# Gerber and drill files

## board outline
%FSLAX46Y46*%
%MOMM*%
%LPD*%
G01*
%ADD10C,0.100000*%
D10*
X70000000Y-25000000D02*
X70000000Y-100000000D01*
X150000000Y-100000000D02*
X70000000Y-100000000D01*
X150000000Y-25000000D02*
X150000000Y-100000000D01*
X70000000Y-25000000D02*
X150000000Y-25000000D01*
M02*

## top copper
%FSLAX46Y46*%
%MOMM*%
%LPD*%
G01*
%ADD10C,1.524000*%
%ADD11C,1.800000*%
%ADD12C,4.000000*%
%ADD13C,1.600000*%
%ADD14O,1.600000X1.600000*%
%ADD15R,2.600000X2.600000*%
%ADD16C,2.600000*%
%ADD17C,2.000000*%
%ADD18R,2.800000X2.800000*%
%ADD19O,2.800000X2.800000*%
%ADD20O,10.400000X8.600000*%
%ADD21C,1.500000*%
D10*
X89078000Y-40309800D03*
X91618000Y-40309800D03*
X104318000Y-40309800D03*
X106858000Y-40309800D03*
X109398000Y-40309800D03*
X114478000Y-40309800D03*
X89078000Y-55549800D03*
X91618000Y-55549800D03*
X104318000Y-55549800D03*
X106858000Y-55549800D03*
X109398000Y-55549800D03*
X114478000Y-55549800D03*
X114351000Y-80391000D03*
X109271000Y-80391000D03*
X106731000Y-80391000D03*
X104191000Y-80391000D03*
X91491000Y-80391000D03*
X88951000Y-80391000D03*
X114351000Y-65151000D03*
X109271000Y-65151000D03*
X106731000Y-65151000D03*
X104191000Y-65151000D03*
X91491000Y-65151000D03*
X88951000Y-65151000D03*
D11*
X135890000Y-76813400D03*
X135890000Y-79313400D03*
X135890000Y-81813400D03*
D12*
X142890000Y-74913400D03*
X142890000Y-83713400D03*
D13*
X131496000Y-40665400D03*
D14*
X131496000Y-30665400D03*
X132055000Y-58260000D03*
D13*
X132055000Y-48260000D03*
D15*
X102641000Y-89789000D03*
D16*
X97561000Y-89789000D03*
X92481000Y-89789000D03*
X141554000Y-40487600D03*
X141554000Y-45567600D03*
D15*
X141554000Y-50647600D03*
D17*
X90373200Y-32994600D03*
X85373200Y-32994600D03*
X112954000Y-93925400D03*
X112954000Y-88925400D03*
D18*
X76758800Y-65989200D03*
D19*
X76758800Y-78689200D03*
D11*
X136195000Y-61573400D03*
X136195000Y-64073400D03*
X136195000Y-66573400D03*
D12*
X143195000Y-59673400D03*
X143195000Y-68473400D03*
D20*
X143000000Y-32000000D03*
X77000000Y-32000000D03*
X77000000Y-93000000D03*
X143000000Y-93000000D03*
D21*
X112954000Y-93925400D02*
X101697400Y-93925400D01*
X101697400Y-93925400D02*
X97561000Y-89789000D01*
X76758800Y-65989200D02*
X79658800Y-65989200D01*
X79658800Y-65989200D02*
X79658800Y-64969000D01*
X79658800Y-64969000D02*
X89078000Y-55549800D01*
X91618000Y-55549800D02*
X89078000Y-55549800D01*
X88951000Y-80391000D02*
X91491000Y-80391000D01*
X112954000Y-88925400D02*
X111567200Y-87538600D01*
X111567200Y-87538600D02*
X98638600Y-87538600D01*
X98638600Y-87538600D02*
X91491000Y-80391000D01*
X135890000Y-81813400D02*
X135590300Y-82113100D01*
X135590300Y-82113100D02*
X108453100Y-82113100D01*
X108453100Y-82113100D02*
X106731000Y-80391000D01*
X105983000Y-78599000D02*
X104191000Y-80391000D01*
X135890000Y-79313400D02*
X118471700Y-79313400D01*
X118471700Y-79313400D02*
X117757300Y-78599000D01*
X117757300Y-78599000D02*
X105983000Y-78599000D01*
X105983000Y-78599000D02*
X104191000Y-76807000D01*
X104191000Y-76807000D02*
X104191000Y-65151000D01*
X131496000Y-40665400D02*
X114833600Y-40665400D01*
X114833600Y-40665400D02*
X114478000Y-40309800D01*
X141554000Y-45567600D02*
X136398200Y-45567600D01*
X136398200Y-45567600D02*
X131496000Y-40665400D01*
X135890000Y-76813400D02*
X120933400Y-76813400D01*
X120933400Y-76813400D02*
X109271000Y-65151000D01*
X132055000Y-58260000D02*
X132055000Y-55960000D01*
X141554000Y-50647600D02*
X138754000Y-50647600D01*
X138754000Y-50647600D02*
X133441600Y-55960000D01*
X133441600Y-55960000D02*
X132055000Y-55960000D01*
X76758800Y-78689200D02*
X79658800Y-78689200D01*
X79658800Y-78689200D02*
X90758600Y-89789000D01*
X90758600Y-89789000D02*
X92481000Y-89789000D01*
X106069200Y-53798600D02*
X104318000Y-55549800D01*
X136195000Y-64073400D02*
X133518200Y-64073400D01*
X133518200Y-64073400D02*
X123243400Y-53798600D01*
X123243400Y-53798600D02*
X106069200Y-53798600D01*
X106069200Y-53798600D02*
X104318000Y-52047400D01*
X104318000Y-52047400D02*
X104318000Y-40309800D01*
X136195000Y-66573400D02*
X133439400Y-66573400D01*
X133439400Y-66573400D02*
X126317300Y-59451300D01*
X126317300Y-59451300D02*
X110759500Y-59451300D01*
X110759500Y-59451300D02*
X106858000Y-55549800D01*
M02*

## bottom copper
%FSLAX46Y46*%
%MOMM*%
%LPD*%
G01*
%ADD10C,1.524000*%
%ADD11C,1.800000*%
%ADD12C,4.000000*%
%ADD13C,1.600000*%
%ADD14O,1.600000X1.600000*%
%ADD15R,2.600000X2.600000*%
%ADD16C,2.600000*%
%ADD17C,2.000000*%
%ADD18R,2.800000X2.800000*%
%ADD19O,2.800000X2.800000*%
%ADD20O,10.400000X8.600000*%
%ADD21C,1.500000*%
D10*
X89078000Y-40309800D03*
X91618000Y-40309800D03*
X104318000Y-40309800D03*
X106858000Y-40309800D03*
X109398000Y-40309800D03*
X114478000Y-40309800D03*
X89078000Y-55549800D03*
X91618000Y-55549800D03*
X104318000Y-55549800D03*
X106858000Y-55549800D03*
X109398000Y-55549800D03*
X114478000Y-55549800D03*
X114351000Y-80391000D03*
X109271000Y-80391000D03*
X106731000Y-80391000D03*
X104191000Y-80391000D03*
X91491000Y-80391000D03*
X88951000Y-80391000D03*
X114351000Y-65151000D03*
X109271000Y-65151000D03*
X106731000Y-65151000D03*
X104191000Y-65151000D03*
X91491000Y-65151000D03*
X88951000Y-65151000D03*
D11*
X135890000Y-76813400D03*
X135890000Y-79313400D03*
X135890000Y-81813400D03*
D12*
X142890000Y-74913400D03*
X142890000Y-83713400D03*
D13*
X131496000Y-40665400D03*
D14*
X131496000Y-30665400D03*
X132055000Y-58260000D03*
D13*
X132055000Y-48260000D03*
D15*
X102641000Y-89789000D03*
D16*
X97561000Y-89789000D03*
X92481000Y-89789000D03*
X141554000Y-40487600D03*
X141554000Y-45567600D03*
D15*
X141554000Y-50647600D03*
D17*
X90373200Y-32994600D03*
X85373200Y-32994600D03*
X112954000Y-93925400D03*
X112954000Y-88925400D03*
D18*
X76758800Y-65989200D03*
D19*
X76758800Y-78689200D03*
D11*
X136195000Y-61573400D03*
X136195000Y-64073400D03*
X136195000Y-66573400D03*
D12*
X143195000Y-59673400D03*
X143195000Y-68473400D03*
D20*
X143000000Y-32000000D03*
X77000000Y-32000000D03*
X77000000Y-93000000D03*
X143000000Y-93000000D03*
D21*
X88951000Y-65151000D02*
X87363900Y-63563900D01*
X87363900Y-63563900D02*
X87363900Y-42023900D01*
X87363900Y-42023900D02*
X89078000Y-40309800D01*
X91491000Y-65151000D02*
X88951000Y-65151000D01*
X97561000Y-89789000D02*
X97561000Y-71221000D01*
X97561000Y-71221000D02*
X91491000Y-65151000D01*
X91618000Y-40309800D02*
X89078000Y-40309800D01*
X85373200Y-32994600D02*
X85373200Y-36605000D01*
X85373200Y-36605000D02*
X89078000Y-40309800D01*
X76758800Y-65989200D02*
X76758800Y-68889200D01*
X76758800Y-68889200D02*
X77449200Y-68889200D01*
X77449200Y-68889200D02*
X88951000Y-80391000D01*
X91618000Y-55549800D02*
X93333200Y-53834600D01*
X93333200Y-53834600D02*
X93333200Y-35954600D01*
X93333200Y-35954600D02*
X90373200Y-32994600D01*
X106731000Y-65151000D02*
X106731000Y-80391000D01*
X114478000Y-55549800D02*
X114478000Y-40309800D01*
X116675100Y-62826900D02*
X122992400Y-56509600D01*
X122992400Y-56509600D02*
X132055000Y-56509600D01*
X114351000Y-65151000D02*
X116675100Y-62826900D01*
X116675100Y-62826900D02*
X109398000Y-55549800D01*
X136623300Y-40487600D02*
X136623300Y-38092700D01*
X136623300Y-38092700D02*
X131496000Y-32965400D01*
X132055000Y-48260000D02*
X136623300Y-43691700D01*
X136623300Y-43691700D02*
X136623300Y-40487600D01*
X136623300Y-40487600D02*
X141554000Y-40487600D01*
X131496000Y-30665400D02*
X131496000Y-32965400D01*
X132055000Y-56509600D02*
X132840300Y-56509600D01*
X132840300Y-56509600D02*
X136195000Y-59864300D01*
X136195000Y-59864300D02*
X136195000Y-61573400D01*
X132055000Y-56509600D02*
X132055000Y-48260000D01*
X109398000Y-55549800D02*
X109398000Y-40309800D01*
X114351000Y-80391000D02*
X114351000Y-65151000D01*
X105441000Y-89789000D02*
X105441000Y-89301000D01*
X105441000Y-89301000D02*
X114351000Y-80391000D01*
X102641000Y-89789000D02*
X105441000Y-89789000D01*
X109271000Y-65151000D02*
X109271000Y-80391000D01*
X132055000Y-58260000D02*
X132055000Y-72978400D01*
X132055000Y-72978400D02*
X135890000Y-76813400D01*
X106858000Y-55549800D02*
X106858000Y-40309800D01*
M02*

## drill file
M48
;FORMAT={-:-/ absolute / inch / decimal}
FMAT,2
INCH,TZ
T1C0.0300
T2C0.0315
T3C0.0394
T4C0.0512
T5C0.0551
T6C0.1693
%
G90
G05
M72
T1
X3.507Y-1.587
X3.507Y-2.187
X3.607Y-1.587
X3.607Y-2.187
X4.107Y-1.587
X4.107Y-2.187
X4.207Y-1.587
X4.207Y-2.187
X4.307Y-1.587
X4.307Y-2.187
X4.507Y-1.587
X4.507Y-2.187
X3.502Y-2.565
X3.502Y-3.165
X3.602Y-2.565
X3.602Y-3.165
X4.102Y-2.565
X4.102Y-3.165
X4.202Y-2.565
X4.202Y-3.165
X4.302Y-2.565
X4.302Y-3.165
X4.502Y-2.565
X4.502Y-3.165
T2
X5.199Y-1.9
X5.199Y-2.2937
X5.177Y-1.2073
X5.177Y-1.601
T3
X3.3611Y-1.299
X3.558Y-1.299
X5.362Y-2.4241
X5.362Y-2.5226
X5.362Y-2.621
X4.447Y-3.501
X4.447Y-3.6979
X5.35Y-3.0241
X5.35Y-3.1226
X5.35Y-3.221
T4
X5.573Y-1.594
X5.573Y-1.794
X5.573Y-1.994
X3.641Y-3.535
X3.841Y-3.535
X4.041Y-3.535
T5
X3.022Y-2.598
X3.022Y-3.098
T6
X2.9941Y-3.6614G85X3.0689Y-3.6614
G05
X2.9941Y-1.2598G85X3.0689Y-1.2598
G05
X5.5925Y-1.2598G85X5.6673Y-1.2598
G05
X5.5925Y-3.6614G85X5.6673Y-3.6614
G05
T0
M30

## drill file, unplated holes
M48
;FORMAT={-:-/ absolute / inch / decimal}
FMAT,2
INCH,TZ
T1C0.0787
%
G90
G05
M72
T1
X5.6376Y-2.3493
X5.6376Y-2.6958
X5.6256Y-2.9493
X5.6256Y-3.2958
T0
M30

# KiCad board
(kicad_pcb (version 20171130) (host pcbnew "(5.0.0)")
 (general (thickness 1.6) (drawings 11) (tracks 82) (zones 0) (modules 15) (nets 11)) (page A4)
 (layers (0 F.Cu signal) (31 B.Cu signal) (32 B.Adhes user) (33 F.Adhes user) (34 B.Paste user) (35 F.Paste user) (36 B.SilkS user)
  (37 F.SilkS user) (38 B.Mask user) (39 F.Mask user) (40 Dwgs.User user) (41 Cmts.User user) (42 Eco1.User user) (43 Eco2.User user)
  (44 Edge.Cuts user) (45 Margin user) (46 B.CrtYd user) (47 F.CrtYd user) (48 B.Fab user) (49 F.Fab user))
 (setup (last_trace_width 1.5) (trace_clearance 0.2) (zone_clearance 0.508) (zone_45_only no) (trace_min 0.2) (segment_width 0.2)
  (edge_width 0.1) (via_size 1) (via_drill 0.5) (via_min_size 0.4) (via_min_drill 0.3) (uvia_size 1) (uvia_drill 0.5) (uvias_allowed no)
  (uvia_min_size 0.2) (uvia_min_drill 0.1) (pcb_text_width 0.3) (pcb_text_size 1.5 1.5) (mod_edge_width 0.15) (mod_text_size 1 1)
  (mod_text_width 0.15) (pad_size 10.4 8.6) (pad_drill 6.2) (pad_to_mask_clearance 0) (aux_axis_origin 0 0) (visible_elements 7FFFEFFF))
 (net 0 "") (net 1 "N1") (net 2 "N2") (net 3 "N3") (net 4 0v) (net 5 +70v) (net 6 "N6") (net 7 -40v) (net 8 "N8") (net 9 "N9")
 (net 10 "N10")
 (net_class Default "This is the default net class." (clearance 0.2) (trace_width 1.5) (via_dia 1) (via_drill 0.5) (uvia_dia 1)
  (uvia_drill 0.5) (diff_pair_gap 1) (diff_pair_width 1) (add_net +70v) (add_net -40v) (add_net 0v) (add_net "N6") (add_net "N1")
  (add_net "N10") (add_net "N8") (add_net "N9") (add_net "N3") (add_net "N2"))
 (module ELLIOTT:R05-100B (layer F.Cu) (at 101.778 47.9298)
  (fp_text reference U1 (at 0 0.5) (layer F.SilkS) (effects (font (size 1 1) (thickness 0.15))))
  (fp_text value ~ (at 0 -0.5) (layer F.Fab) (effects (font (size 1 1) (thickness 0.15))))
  (pad 2 thru_hole circle (at -12.7 -7.62) (size 1.524 1.524) (drill 0.762) (layers *.Cu *.Mask) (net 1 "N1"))
  (pad 3 thru_hole circle (at -10.16 -7.62) (size 1.524 1.524) (drill 0.762) (layers *.Cu *.Mask) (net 1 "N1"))
  (pad 8 thru_hole circle (at 2.54 -7.62) (size 1.524 1.524) (drill 0.762) (layers *.Cu *.Mask) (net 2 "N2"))
  (pad 9 thru_hole circle (at 5.08 -7.62) (size 1.524 1.524) (drill 0.762) (layers *.Cu *.Mask) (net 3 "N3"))
  (pad 10 thru_hole circle (at 7.62 -7.62) (size 1.524 1.524) (drill 0.762) (layers *.Cu *.Mask) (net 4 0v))
  (pad 12 thru_hole circle (at 12.7 -7.62) (size 1.524 1.524) (drill 0.762) (layers *.Cu *.Mask) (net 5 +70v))
  (pad 22 thru_hole circle (at -12.7 7.62) (size 1.524 1.524) (drill 0.762) (layers *.Cu *.Mask) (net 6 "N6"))
  (pad 23 thru_hole circle (at -10.16 7.62) (size 1.524 1.524) (drill 0.762) (layers *.Cu *.Mask) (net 6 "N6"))
  (pad 17 thru_hole circle (at 2.54 7.62) (size 1.524 1.524) (drill 0.762) (layers *.Cu *.Mask) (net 2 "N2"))
  (pad 16 thru_hole circle (at 5.08 7.62) (size 1.524 1.524) (drill 0.762) (layers *.Cu *.Mask) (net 3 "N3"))
  (pad 15 thru_hole circle (at 7.62 7.62) (size 1.524 1.524) (drill 0.762) (layers *.Cu *.Mask) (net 4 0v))
  (pad 13 thru_hole circle (at 12.7 7.62) (size 1.524 1.524) (drill 0.762) (layers *.Cu *.Mask) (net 5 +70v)))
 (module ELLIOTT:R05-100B (layer F.Cu) (at 101.651 72.771)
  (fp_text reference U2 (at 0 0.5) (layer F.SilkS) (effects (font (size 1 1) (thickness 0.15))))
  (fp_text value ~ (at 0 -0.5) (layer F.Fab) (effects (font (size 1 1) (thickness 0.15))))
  (pad 13 thru_hole circle (at 12.7 7.62) (size 1.524 1.524) (drill 0.762) (layers *.Cu *.Mask) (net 4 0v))
  (pad 15 thru_hole circle (at 7.62 7.62) (size 1.524 1.524) (drill 0.762) (layers *.Cu *.Mask) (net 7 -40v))
  (pad 16 thru_hole circle (at 5.08 7.62) (size 1.524 1.524) (drill 0.762) (layers *.Cu *.Mask) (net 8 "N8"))
  (pad 17 thru_hole circle (at 2.54 7.62) (size 1.524 1.524) (drill 0.762) (layers *.Cu *.Mask) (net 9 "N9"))
  (pad 23 thru_hole circle (at -10.16 7.62) (size 1.524 1.524) (drill 0.762) (layers *.Cu *.Mask) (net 6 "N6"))
  (pad 22 thru_hole circle (at -12.7 7.62) (size 1.524 1.524) (drill 0.762) (layers *.Cu *.Mask) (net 6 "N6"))
  (pad 12 thru_hole circle (at 12.7 -7.62) (size 1.524 1.524) (drill 0.762) (layers *.Cu *.Mask) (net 4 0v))
  (pad 10 thru_hole circle (at 7.62 -7.62) (size 1.524 1.524) (drill 0.762) (layers *.Cu *.Mask) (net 7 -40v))
  (pad 9 thru_hole circle (at 5.08 -7.62) (size 1.524 1.524) (drill 0.762) (layers *.Cu *.Mask) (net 8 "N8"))
  (pad 8 thru_hole circle (at 2.54 -7.62) (size 1.524 1.524) (drill 0.762) (layers *.Cu *.Mask) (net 9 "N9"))
  (pad 3 thru_hole circle (at -10.16 -7.62) (size 1.524 1.524) (drill 0.762) (layers *.Cu *.Mask) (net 1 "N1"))
  (pad 2 thru_hole circle (at -12.7 -7.62) (size 1.524 1.524) (drill 0.762) (layers *.Cu *.Mask) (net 1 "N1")))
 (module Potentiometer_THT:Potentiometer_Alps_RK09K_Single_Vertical (layer F.Cu) (at 135.89 81.8134)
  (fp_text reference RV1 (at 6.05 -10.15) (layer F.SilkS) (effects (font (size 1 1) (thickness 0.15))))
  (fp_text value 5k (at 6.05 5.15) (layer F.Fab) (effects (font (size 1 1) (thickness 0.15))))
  (pad 3 thru_hole circle (at 0 -5) (size 1.8 1.8) (drill 1) (layers *.Cu *.Mask) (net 7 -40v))
  (pad 2 thru_hole circle (at 0 -2.5) (size 1.8 1.8) (drill 1) (layers *.Cu *.Mask) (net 9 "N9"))
  (pad 1 thru_hole circle (at 0 0) (size 1.8 1.8) (drill 1) (layers *.Cu *.Mask) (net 8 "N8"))
  (pad "" np_thru_hole circle (at 7 -6.9) (size 4 4) (drill 2) (layers *.Cu *.Mask))
  (pad "" np_thru_hole circle (at 7 1.9) (size 4 4) (drill 2) (layers *.Cu *.Mask)))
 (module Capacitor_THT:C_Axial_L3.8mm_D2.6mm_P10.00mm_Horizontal (layer F.Cu) (at 131.496 40.6654 90)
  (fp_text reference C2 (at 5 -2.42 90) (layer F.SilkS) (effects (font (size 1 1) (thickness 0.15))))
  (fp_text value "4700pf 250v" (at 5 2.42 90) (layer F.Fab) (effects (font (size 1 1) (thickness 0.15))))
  (pad 1 thru_hole circle (at 0 0 90) (size 1.6 1.6) (drill 0.8) (layers *.Cu *.Mask) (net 5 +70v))
  (pad 2 thru_hole oval (at 10 0 90) (size 1.6 1.6) (drill 0.8) (layers *.Cu *.Mask) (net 4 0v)))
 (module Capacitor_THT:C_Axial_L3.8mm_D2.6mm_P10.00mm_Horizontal (layer F.Cu) (at 132.055 48.26 270)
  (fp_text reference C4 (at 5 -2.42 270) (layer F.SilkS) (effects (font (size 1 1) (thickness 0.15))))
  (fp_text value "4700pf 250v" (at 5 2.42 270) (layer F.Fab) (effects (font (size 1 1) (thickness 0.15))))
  (pad 2 thru_hole oval (at 10 0 270) (size 1.6 1.6) (drill 0.8) (layers *.Cu *.Mask) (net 7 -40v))
  (pad 1 thru_hole circle (at 0 0 270) (size 1.6 1.6) (drill 0.8) (layers *.Cu *.Mask) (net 4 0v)))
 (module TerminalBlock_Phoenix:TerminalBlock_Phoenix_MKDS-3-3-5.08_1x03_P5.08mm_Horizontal (layer F.Cu) (at 102.641 89.789 180)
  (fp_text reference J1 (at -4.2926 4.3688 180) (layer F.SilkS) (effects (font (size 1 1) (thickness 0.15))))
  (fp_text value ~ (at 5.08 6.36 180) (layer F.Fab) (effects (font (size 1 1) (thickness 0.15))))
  (pad 1 thru_hole rect (at 0 0 180) (size 2.6 2.6) (drill 1.3) (layers *.Cu *.Mask) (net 4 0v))
  (pad 2 thru_hole circle (at 5.08 0 180) (size 2.6 2.6) (drill 1.3) (layers *.Cu *.Mask) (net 1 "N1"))
  (pad 3 thru_hole circle (at 10.16 0 180) (size 2.6 2.6) (drill 1.3) (layers *.Cu *.Mask) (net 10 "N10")))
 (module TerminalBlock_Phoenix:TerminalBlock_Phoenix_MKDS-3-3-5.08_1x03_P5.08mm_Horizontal (layer F.Cu) (at 141.554 50.6476 90)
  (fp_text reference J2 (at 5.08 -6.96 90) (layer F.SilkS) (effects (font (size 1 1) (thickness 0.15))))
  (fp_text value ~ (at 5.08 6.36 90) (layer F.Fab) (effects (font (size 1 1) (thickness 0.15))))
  (pad 3 thru_hole circle (at 10.16 0 90) (size 2.6 2.6) (drill 1.3) (layers *.Cu *.Mask) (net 4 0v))
  (pad 2 thru_hole circle (at 5.08 0 90) (size 2.6 2.6) (drill 1.3) (layers *.Cu *.Mask) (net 5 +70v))
  (pad 1 thru_hole rect (at 0 0 90) (size 2.6 2.6) (drill 1.3) (layers *.Cu *.Mask) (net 7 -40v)))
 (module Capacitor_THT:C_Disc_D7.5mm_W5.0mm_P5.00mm (layer F.Cu) (at 90.3732 32.9946 180)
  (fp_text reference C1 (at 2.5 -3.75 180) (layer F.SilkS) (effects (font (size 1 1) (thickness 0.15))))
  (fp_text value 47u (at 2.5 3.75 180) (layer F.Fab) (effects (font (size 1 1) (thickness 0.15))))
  (pad 1 thru_hole circle (at 0 0 180) (size 2 2) (drill 1) (layers *.Cu *.Mask) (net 6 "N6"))
  (pad 2 thru_hole circle (at 5 0 180) (size 2 2) (drill 1) (layers *.Cu *.Mask) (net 1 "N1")))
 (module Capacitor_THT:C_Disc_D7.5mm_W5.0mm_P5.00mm (layer F.Cu) (at 112.954 88.9254 270)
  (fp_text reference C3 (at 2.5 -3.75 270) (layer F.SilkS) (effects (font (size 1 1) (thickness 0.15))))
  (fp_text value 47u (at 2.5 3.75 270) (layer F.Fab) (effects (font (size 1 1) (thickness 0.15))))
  (pad 2 thru_hole circle (at 5 0 270) (size 2 2) (drill 1) (layers *.Cu *.Mask) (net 1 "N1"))
  (pad 1 thru_hole circle (at 0 0 270) (size 2 2) (drill 1) (layers *.Cu *.Mask) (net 6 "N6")))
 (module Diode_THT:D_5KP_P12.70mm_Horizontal (layer F.Cu) (at 76.7588 65.9892 270)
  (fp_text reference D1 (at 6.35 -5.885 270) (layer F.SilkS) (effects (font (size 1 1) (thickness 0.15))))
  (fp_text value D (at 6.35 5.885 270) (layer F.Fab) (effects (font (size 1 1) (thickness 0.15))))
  (pad 1 thru_hole rect (at 0 0 270) (size 2.8 2.8) (drill 1.4) (layers *.Cu *.Mask) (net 6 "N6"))
  (pad 2 thru_hole oval (at 12.7 0 270) (size 2.8 2.8) (drill 1.4) (layers *.Cu *.Mask) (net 10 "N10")))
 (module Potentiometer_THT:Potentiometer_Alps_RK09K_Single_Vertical (layer F.Cu) (at 136.195 66.5734)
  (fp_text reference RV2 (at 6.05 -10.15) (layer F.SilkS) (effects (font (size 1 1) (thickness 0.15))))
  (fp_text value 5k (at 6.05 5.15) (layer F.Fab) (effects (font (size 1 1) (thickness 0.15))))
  (pad 3 thru_hole circle (at 0 -5) (size 1.8 1.8) (drill 1) (layers *.Cu *.Mask) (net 4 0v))
  (pad 2 thru_hole circle (at 0 -2.5) (size 1.8 1.8) (drill 1) (layers *.Cu *.Mask) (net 2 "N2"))
  (pad 1 thru_hole circle (at 0 0) (size 1.8 1.8) (drill 1) (layers *.Cu *.Mask) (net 3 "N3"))
  (pad "" np_thru_hole circle (at 7 -6.9) (size 4 4) (drill 2) (layers *.Cu *.Mask))
  (pad "" np_thru_hole circle (at 7 1.9) (size 4 4) (drill 2) (layers *.Cu *.Mask)))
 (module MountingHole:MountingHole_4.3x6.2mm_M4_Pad (layer F.Cu) (at 143 32)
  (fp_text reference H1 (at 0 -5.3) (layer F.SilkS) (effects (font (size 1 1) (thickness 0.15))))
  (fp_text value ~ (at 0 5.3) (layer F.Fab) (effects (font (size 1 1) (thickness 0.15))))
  (pad 1 thru_hole oval (at 0 0) (size 10.4 8.6) (drill oval 6.2 4.3) (layers *.Cu *.Mask)))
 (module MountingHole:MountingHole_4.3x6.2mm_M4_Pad (layer F.Cu) (at 77 32)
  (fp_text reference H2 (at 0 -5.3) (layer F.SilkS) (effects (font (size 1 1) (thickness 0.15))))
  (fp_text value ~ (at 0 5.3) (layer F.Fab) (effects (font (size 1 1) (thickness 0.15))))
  (pad 1 thru_hole oval (at 0 0) (size 10.4 8.6) (drill oval 6.2 4.3) (layers *.Cu *.Mask)))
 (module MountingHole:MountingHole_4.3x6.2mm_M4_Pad (layer F.Cu) (at 77 93)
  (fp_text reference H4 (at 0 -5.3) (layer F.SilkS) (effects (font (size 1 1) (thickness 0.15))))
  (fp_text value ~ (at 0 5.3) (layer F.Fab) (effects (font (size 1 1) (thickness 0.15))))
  (pad 1 thru_hole oval (at 0 0) (size 10.4 8.6) (drill oval 6.2 4.3) (layers *.Cu *.Mask)))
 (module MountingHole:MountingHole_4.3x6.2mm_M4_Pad (layer F.Cu) (at 143 93)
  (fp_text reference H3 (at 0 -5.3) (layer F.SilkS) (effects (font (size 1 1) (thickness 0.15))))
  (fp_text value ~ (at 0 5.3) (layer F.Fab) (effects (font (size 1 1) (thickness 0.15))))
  (pad 1 thru_hole oval (at 0 0) (size 10.4 8.6) (drill oval 6.2 4.3) (layers *.Cu *.Mask)))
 (gr_line (start 70 25) (end 70 100) (layer Edge.Cuts) (width 0.1))
 (gr_line (start 150 100) (end 70 100) (layer Edge.Cuts) (width 0.1))
 (gr_line (start 150 25) (end 150 100) (layer Edge.Cuts) (width 0.1))
 (gr_line (start 70 25) (end 150 25) (layer Edge.Cuts) (width 0.1))
 (segment (start 88.951 65.151) (end 87.3639 63.5639) (width 1.5) (layer B.Cu) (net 1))
 (segment (start 87.3639 63.5639) (end 87.3639 42.0239) (width 1.5) (layer B.Cu) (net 1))
 (segment (start 87.3639 42.0239) (end 89.078 40.3098) (width 1.5) (layer B.Cu) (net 1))
 (segment (start 91.491 65.151) (end 88.951 65.151) (width 1.5) (layer B.Cu) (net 1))
 (segment (start 97.561 89.789) (end 97.561 71.221) (width 1.5) (layer B.Cu) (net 1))
 (segment (start 97.561 71.221) (end 91.491 65.151) (width 1.5) (layer B.Cu) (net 1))
 (segment (start 91.618 40.3098) (end 89.078 40.3098) (width 1.5) (layer B.Cu) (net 1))
 (segment (start 85.3732 32.9946) (end 85.3732 36.605) (width 1.5) (layer B.Cu) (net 1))
 (segment (start 85.3732 36.605) (end 89.078 40.3098) (width 1.5) (layer B.Cu) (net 1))
 (segment (start 112.954 93.9254) (end 101.6974 93.9254) (width 1.5) (layer F.Cu) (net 1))
 (segment (start 101.6974 93.9254) (end 97.561 89.789) (width 1.5) (layer F.Cu) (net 1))
 (segment (start 76.7588 65.9892) (end 76.7588 68.8892) (width 1.5) (layer B.Cu) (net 6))
 (segment (start 76.7588 68.8892) (end 77.4492 68.8892) (width 1.5) (layer B.Cu) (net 6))
 (segment (start 77.4492 68.8892) (end 88.951 80.391) (width 1.5) (layer B.Cu) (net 6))
 (segment (start 91.618 55.5498) (end 93.3332 53.8346) (width 1.5) (layer B.Cu) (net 6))
 (segment (start 93.3332 53.8346) (end 93.3332 35.9546) (width 1.5) (layer B.Cu) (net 6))
 (segment (start 93.3332 35.9546) (end 90.3732 32.9946) (width 1.5) (layer B.Cu) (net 6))
 (segment (start 76.7588 65.9892) (end 79.6588 65.9892) (width 1.5) (layer F.Cu) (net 6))
 (segment (start 79.6588 65.9892) (end 79.6588 64.969) (width 1.5) (layer F.Cu) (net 6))
 (segment (start 79.6588 64.969) (end 89.078 55.5498) (width 1.5) (layer F.Cu) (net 6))
 (segment (start 91.618 55.5498) (end 89.078 55.5498) (width 1.5) (layer F.Cu) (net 6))
 (segment (start 88.951 80.391) (end 91.491 80.391) (width 1.5) (layer F.Cu) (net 6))
 (segment (start 112.954 88.9254) (end 111.5672 87.5386) (width 1.5) (layer F.Cu) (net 6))
 (segment (start 111.5672 87.5386) (end 98.6386 87.5386) (width 1.5) (layer F.Cu) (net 6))
 (segment (start 98.6386 87.5386) (end 91.491 80.391) (width 1.5) (layer F.Cu) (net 6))
 (segment (start 106.731 65.151) (end 106.731 80.391) (width 1.5) (layer B.Cu) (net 8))
 (segment (start 135.89 81.8134) (end 135.5903 82.1131) (width 1.5) (layer F.Cu) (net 8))
 (segment (start 135.5903 82.1131) (end 108.4531 82.1131) (width 1.5) (layer F.Cu) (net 8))
 (segment (start 108.4531 82.1131) (end 106.731 80.391) (width 1.5) (layer F.Cu) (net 8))
 (segment (start 105.983 78.599) (end 104.191 80.391) (width 1.5) (layer F.Cu) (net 9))
 (segment (start 135.89 79.3134) (end 118.4717 79.3134) (width 1.5) (layer F.Cu) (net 9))
 (segment (start 118.4717 79.3134) (end 117.7573 78.599) (width 1.5) (layer F.Cu) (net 9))
 (segment (start 117.7573 78.599) (end 105.983 78.599) (width 1.5) (layer F.Cu) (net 9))
 (segment (start 105.983 78.599) (end 104.191 76.807) (width 1.5) (layer F.Cu) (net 9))
 (segment (start 104.191 76.807) (end 104.191 65.151) (width 1.5) (layer F.Cu) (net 9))
 (segment (start 114.478 55.5498) (end 114.478 40.3098) (width 1.5) (layer B.Cu) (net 5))
 (segment (start 131.496 40.6654) (end 114.8336 40.6654) (width 1.5) (layer F.Cu) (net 5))
 (segment (start 114.8336 40.6654) (end 114.478 40.3098) (width 1.5) (layer F.Cu) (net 5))
 (segment (start 141.554 45.5676) (end 136.3982 45.5676) (width 1.5) (layer F.Cu) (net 5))
 (segment (start 136.3982 45.5676) (end 131.496 40.6654) (width 1.5) (layer F.Cu) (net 5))
 (segment (start 116.6751 62.8269) (end 122.9924 56.5096) (width 1.5) (layer B.Cu) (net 4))
 (segment (start 122.9924 56.5096) (end 132.055 56.5096) (width 1.5) (layer B.Cu) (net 4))
 (segment (start 114.351 65.151) (end 116.6751 62.8269) (width 1.5) (layer B.Cu) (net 4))
 (segment (start 116.6751 62.8269) (end 109.398 55.5498) (width 1.5) (layer B.Cu) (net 4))
 (segment (start 136.6233 40.4876) (end 136.6233 38.0927) (width 1.5) (layer B.Cu) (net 4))
 (segment (start 136.6233 38.0927) (end 131.496 32.9654) (width 1.5) (layer B.Cu) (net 4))
 (segment (start 132.055 48.26) (end 136.6233 43.6917) (width 1.5) (layer B.Cu) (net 4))
 (segment (start 136.6233 43.6917) (end 136.6233 40.4876) (width 1.5) (layer B.Cu) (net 4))
 (segment (start 136.6233 40.4876) (end 141.554 40.4876) (width 1.5) (layer B.Cu) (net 4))
 (segment (start 131.496 30.6654) (end 131.496 32.9654) (width 1.5) (layer B.Cu) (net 4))
 (segment (start 132.055 56.5096) (end 132.8403 56.5096) (width 1.5) (layer B.Cu) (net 4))
 (segment (start 132.8403 56.5096) (end 136.195 59.8643) (width 1.5) (layer B.Cu) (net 4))
 (segment (start 136.195 59.8643) (end 136.195 61.5734) (width 1.5) (layer B.Cu) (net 4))
 (segment (start 132.055 56.5096) (end 132.055 48.26) (width 1.5) (layer B.Cu) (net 4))
 (segment (start 109.398 55.5498) (end 109.398 40.3098) (width 1.5) (layer B.Cu) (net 4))
 (segment (start 114.351 80.391) (end 114.351 65.151) (width 1.5) (layer B.Cu) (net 4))
 (segment (start 105.441 89.789) (end 105.441 89.301) (width 1.5) (layer B.Cu) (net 4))
 (segment (start 105.441 89.301) (end 114.351 80.391) (width 1.5) (layer B.Cu) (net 4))
 (segment (start 102.641 89.789) (end 105.441 89.789) (width 1.5) (layer B.Cu) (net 4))
 (segment (start 109.271 65.151) (end 109.271 80.391) (width 1.5) (layer B.Cu) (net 7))
 (segment (start 135.89 76.8134) (end 120.9334 76.8134) (width 1.5) (layer F.Cu) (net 7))
 (segment (start 120.9334 76.8134) (end 109.271 65.151) (width 1.5) (layer F.Cu) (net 7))
 (segment (start 132.055 58.26) (end 132.055 72.9784) (width 1.5) (layer B.Cu) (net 7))
 (segment (start 132.055 72.9784) (end 135.89 76.8134) (width 1.5) (layer B.Cu) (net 7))
 (segment (start 132.055 58.26) (end 132.055 55.96) (width 1.5) (layer F.Cu) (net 7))
 (segment (start 141.554 50.6476) (end 138.754 50.6476) (width 1.5) (layer F.Cu) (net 7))
 (segment (start 138.754 50.6476) (end 133.4416 55.96) (width 1.5) (layer F.Cu) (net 7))
 (segment (start 133.4416 55.96) (end 132.055 55.96) (width 1.5) (layer F.Cu) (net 7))
 (segment (start 76.7588 78.6892) (end 79.6588 78.6892) (width 1.5) (layer F.Cu) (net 10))
 (segment (start 79.6588 78.6892) (end 90.7586 89.789) (width 1.5) (layer F.Cu) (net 10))
 (segment (start 90.7586 89.789) (end 92.481 89.789) (width 1.5) (layer F.Cu) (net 10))
 (segment (start 106.0692 53.7986) (end 104.318 55.5498) (width 1.5) (layer F.Cu) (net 2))
 (segment (start 136.195 64.0734) (end 133.5182 64.0734) (width 1.5) (layer F.Cu) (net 2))
 (segment (start 133.5182 64.0734) (end 123.2434 53.7986) (width 1.5) (layer F.Cu) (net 2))
 (segment (start 123.2434 53.7986) (end 106.0692 53.7986) (width 1.5) (layer F.Cu) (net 2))
 (segment (start 106.0692 53.7986) (end 104.318 52.0474) (width 1.5) (layer F.Cu) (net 2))
 (segment (start 104.318 52.0474) (end 104.318 40.3098) (width 1.5) (layer F.Cu) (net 2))
 (segment (start 106.858 55.5498) (end 106.858 40.3098) (width 1.5) (layer B.Cu) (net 3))
 (segment (start 136.195 66.5734) (end 133.4394 66.5734) (width 1.5) (layer F.Cu) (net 3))
 (segment (start 133.4394 66.5734) (end 126.3173 59.4513) (width 1.5) (layer F.Cu) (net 3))
 (segment (start 126.3173 59.4513) (end 110.7595 59.4513) (width 1.5) (layer F.Cu) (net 3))
 (segment (start 110.7595 59.4513) (end 106.858 55.5498) (width 1.5) (layer F.Cu) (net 3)))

